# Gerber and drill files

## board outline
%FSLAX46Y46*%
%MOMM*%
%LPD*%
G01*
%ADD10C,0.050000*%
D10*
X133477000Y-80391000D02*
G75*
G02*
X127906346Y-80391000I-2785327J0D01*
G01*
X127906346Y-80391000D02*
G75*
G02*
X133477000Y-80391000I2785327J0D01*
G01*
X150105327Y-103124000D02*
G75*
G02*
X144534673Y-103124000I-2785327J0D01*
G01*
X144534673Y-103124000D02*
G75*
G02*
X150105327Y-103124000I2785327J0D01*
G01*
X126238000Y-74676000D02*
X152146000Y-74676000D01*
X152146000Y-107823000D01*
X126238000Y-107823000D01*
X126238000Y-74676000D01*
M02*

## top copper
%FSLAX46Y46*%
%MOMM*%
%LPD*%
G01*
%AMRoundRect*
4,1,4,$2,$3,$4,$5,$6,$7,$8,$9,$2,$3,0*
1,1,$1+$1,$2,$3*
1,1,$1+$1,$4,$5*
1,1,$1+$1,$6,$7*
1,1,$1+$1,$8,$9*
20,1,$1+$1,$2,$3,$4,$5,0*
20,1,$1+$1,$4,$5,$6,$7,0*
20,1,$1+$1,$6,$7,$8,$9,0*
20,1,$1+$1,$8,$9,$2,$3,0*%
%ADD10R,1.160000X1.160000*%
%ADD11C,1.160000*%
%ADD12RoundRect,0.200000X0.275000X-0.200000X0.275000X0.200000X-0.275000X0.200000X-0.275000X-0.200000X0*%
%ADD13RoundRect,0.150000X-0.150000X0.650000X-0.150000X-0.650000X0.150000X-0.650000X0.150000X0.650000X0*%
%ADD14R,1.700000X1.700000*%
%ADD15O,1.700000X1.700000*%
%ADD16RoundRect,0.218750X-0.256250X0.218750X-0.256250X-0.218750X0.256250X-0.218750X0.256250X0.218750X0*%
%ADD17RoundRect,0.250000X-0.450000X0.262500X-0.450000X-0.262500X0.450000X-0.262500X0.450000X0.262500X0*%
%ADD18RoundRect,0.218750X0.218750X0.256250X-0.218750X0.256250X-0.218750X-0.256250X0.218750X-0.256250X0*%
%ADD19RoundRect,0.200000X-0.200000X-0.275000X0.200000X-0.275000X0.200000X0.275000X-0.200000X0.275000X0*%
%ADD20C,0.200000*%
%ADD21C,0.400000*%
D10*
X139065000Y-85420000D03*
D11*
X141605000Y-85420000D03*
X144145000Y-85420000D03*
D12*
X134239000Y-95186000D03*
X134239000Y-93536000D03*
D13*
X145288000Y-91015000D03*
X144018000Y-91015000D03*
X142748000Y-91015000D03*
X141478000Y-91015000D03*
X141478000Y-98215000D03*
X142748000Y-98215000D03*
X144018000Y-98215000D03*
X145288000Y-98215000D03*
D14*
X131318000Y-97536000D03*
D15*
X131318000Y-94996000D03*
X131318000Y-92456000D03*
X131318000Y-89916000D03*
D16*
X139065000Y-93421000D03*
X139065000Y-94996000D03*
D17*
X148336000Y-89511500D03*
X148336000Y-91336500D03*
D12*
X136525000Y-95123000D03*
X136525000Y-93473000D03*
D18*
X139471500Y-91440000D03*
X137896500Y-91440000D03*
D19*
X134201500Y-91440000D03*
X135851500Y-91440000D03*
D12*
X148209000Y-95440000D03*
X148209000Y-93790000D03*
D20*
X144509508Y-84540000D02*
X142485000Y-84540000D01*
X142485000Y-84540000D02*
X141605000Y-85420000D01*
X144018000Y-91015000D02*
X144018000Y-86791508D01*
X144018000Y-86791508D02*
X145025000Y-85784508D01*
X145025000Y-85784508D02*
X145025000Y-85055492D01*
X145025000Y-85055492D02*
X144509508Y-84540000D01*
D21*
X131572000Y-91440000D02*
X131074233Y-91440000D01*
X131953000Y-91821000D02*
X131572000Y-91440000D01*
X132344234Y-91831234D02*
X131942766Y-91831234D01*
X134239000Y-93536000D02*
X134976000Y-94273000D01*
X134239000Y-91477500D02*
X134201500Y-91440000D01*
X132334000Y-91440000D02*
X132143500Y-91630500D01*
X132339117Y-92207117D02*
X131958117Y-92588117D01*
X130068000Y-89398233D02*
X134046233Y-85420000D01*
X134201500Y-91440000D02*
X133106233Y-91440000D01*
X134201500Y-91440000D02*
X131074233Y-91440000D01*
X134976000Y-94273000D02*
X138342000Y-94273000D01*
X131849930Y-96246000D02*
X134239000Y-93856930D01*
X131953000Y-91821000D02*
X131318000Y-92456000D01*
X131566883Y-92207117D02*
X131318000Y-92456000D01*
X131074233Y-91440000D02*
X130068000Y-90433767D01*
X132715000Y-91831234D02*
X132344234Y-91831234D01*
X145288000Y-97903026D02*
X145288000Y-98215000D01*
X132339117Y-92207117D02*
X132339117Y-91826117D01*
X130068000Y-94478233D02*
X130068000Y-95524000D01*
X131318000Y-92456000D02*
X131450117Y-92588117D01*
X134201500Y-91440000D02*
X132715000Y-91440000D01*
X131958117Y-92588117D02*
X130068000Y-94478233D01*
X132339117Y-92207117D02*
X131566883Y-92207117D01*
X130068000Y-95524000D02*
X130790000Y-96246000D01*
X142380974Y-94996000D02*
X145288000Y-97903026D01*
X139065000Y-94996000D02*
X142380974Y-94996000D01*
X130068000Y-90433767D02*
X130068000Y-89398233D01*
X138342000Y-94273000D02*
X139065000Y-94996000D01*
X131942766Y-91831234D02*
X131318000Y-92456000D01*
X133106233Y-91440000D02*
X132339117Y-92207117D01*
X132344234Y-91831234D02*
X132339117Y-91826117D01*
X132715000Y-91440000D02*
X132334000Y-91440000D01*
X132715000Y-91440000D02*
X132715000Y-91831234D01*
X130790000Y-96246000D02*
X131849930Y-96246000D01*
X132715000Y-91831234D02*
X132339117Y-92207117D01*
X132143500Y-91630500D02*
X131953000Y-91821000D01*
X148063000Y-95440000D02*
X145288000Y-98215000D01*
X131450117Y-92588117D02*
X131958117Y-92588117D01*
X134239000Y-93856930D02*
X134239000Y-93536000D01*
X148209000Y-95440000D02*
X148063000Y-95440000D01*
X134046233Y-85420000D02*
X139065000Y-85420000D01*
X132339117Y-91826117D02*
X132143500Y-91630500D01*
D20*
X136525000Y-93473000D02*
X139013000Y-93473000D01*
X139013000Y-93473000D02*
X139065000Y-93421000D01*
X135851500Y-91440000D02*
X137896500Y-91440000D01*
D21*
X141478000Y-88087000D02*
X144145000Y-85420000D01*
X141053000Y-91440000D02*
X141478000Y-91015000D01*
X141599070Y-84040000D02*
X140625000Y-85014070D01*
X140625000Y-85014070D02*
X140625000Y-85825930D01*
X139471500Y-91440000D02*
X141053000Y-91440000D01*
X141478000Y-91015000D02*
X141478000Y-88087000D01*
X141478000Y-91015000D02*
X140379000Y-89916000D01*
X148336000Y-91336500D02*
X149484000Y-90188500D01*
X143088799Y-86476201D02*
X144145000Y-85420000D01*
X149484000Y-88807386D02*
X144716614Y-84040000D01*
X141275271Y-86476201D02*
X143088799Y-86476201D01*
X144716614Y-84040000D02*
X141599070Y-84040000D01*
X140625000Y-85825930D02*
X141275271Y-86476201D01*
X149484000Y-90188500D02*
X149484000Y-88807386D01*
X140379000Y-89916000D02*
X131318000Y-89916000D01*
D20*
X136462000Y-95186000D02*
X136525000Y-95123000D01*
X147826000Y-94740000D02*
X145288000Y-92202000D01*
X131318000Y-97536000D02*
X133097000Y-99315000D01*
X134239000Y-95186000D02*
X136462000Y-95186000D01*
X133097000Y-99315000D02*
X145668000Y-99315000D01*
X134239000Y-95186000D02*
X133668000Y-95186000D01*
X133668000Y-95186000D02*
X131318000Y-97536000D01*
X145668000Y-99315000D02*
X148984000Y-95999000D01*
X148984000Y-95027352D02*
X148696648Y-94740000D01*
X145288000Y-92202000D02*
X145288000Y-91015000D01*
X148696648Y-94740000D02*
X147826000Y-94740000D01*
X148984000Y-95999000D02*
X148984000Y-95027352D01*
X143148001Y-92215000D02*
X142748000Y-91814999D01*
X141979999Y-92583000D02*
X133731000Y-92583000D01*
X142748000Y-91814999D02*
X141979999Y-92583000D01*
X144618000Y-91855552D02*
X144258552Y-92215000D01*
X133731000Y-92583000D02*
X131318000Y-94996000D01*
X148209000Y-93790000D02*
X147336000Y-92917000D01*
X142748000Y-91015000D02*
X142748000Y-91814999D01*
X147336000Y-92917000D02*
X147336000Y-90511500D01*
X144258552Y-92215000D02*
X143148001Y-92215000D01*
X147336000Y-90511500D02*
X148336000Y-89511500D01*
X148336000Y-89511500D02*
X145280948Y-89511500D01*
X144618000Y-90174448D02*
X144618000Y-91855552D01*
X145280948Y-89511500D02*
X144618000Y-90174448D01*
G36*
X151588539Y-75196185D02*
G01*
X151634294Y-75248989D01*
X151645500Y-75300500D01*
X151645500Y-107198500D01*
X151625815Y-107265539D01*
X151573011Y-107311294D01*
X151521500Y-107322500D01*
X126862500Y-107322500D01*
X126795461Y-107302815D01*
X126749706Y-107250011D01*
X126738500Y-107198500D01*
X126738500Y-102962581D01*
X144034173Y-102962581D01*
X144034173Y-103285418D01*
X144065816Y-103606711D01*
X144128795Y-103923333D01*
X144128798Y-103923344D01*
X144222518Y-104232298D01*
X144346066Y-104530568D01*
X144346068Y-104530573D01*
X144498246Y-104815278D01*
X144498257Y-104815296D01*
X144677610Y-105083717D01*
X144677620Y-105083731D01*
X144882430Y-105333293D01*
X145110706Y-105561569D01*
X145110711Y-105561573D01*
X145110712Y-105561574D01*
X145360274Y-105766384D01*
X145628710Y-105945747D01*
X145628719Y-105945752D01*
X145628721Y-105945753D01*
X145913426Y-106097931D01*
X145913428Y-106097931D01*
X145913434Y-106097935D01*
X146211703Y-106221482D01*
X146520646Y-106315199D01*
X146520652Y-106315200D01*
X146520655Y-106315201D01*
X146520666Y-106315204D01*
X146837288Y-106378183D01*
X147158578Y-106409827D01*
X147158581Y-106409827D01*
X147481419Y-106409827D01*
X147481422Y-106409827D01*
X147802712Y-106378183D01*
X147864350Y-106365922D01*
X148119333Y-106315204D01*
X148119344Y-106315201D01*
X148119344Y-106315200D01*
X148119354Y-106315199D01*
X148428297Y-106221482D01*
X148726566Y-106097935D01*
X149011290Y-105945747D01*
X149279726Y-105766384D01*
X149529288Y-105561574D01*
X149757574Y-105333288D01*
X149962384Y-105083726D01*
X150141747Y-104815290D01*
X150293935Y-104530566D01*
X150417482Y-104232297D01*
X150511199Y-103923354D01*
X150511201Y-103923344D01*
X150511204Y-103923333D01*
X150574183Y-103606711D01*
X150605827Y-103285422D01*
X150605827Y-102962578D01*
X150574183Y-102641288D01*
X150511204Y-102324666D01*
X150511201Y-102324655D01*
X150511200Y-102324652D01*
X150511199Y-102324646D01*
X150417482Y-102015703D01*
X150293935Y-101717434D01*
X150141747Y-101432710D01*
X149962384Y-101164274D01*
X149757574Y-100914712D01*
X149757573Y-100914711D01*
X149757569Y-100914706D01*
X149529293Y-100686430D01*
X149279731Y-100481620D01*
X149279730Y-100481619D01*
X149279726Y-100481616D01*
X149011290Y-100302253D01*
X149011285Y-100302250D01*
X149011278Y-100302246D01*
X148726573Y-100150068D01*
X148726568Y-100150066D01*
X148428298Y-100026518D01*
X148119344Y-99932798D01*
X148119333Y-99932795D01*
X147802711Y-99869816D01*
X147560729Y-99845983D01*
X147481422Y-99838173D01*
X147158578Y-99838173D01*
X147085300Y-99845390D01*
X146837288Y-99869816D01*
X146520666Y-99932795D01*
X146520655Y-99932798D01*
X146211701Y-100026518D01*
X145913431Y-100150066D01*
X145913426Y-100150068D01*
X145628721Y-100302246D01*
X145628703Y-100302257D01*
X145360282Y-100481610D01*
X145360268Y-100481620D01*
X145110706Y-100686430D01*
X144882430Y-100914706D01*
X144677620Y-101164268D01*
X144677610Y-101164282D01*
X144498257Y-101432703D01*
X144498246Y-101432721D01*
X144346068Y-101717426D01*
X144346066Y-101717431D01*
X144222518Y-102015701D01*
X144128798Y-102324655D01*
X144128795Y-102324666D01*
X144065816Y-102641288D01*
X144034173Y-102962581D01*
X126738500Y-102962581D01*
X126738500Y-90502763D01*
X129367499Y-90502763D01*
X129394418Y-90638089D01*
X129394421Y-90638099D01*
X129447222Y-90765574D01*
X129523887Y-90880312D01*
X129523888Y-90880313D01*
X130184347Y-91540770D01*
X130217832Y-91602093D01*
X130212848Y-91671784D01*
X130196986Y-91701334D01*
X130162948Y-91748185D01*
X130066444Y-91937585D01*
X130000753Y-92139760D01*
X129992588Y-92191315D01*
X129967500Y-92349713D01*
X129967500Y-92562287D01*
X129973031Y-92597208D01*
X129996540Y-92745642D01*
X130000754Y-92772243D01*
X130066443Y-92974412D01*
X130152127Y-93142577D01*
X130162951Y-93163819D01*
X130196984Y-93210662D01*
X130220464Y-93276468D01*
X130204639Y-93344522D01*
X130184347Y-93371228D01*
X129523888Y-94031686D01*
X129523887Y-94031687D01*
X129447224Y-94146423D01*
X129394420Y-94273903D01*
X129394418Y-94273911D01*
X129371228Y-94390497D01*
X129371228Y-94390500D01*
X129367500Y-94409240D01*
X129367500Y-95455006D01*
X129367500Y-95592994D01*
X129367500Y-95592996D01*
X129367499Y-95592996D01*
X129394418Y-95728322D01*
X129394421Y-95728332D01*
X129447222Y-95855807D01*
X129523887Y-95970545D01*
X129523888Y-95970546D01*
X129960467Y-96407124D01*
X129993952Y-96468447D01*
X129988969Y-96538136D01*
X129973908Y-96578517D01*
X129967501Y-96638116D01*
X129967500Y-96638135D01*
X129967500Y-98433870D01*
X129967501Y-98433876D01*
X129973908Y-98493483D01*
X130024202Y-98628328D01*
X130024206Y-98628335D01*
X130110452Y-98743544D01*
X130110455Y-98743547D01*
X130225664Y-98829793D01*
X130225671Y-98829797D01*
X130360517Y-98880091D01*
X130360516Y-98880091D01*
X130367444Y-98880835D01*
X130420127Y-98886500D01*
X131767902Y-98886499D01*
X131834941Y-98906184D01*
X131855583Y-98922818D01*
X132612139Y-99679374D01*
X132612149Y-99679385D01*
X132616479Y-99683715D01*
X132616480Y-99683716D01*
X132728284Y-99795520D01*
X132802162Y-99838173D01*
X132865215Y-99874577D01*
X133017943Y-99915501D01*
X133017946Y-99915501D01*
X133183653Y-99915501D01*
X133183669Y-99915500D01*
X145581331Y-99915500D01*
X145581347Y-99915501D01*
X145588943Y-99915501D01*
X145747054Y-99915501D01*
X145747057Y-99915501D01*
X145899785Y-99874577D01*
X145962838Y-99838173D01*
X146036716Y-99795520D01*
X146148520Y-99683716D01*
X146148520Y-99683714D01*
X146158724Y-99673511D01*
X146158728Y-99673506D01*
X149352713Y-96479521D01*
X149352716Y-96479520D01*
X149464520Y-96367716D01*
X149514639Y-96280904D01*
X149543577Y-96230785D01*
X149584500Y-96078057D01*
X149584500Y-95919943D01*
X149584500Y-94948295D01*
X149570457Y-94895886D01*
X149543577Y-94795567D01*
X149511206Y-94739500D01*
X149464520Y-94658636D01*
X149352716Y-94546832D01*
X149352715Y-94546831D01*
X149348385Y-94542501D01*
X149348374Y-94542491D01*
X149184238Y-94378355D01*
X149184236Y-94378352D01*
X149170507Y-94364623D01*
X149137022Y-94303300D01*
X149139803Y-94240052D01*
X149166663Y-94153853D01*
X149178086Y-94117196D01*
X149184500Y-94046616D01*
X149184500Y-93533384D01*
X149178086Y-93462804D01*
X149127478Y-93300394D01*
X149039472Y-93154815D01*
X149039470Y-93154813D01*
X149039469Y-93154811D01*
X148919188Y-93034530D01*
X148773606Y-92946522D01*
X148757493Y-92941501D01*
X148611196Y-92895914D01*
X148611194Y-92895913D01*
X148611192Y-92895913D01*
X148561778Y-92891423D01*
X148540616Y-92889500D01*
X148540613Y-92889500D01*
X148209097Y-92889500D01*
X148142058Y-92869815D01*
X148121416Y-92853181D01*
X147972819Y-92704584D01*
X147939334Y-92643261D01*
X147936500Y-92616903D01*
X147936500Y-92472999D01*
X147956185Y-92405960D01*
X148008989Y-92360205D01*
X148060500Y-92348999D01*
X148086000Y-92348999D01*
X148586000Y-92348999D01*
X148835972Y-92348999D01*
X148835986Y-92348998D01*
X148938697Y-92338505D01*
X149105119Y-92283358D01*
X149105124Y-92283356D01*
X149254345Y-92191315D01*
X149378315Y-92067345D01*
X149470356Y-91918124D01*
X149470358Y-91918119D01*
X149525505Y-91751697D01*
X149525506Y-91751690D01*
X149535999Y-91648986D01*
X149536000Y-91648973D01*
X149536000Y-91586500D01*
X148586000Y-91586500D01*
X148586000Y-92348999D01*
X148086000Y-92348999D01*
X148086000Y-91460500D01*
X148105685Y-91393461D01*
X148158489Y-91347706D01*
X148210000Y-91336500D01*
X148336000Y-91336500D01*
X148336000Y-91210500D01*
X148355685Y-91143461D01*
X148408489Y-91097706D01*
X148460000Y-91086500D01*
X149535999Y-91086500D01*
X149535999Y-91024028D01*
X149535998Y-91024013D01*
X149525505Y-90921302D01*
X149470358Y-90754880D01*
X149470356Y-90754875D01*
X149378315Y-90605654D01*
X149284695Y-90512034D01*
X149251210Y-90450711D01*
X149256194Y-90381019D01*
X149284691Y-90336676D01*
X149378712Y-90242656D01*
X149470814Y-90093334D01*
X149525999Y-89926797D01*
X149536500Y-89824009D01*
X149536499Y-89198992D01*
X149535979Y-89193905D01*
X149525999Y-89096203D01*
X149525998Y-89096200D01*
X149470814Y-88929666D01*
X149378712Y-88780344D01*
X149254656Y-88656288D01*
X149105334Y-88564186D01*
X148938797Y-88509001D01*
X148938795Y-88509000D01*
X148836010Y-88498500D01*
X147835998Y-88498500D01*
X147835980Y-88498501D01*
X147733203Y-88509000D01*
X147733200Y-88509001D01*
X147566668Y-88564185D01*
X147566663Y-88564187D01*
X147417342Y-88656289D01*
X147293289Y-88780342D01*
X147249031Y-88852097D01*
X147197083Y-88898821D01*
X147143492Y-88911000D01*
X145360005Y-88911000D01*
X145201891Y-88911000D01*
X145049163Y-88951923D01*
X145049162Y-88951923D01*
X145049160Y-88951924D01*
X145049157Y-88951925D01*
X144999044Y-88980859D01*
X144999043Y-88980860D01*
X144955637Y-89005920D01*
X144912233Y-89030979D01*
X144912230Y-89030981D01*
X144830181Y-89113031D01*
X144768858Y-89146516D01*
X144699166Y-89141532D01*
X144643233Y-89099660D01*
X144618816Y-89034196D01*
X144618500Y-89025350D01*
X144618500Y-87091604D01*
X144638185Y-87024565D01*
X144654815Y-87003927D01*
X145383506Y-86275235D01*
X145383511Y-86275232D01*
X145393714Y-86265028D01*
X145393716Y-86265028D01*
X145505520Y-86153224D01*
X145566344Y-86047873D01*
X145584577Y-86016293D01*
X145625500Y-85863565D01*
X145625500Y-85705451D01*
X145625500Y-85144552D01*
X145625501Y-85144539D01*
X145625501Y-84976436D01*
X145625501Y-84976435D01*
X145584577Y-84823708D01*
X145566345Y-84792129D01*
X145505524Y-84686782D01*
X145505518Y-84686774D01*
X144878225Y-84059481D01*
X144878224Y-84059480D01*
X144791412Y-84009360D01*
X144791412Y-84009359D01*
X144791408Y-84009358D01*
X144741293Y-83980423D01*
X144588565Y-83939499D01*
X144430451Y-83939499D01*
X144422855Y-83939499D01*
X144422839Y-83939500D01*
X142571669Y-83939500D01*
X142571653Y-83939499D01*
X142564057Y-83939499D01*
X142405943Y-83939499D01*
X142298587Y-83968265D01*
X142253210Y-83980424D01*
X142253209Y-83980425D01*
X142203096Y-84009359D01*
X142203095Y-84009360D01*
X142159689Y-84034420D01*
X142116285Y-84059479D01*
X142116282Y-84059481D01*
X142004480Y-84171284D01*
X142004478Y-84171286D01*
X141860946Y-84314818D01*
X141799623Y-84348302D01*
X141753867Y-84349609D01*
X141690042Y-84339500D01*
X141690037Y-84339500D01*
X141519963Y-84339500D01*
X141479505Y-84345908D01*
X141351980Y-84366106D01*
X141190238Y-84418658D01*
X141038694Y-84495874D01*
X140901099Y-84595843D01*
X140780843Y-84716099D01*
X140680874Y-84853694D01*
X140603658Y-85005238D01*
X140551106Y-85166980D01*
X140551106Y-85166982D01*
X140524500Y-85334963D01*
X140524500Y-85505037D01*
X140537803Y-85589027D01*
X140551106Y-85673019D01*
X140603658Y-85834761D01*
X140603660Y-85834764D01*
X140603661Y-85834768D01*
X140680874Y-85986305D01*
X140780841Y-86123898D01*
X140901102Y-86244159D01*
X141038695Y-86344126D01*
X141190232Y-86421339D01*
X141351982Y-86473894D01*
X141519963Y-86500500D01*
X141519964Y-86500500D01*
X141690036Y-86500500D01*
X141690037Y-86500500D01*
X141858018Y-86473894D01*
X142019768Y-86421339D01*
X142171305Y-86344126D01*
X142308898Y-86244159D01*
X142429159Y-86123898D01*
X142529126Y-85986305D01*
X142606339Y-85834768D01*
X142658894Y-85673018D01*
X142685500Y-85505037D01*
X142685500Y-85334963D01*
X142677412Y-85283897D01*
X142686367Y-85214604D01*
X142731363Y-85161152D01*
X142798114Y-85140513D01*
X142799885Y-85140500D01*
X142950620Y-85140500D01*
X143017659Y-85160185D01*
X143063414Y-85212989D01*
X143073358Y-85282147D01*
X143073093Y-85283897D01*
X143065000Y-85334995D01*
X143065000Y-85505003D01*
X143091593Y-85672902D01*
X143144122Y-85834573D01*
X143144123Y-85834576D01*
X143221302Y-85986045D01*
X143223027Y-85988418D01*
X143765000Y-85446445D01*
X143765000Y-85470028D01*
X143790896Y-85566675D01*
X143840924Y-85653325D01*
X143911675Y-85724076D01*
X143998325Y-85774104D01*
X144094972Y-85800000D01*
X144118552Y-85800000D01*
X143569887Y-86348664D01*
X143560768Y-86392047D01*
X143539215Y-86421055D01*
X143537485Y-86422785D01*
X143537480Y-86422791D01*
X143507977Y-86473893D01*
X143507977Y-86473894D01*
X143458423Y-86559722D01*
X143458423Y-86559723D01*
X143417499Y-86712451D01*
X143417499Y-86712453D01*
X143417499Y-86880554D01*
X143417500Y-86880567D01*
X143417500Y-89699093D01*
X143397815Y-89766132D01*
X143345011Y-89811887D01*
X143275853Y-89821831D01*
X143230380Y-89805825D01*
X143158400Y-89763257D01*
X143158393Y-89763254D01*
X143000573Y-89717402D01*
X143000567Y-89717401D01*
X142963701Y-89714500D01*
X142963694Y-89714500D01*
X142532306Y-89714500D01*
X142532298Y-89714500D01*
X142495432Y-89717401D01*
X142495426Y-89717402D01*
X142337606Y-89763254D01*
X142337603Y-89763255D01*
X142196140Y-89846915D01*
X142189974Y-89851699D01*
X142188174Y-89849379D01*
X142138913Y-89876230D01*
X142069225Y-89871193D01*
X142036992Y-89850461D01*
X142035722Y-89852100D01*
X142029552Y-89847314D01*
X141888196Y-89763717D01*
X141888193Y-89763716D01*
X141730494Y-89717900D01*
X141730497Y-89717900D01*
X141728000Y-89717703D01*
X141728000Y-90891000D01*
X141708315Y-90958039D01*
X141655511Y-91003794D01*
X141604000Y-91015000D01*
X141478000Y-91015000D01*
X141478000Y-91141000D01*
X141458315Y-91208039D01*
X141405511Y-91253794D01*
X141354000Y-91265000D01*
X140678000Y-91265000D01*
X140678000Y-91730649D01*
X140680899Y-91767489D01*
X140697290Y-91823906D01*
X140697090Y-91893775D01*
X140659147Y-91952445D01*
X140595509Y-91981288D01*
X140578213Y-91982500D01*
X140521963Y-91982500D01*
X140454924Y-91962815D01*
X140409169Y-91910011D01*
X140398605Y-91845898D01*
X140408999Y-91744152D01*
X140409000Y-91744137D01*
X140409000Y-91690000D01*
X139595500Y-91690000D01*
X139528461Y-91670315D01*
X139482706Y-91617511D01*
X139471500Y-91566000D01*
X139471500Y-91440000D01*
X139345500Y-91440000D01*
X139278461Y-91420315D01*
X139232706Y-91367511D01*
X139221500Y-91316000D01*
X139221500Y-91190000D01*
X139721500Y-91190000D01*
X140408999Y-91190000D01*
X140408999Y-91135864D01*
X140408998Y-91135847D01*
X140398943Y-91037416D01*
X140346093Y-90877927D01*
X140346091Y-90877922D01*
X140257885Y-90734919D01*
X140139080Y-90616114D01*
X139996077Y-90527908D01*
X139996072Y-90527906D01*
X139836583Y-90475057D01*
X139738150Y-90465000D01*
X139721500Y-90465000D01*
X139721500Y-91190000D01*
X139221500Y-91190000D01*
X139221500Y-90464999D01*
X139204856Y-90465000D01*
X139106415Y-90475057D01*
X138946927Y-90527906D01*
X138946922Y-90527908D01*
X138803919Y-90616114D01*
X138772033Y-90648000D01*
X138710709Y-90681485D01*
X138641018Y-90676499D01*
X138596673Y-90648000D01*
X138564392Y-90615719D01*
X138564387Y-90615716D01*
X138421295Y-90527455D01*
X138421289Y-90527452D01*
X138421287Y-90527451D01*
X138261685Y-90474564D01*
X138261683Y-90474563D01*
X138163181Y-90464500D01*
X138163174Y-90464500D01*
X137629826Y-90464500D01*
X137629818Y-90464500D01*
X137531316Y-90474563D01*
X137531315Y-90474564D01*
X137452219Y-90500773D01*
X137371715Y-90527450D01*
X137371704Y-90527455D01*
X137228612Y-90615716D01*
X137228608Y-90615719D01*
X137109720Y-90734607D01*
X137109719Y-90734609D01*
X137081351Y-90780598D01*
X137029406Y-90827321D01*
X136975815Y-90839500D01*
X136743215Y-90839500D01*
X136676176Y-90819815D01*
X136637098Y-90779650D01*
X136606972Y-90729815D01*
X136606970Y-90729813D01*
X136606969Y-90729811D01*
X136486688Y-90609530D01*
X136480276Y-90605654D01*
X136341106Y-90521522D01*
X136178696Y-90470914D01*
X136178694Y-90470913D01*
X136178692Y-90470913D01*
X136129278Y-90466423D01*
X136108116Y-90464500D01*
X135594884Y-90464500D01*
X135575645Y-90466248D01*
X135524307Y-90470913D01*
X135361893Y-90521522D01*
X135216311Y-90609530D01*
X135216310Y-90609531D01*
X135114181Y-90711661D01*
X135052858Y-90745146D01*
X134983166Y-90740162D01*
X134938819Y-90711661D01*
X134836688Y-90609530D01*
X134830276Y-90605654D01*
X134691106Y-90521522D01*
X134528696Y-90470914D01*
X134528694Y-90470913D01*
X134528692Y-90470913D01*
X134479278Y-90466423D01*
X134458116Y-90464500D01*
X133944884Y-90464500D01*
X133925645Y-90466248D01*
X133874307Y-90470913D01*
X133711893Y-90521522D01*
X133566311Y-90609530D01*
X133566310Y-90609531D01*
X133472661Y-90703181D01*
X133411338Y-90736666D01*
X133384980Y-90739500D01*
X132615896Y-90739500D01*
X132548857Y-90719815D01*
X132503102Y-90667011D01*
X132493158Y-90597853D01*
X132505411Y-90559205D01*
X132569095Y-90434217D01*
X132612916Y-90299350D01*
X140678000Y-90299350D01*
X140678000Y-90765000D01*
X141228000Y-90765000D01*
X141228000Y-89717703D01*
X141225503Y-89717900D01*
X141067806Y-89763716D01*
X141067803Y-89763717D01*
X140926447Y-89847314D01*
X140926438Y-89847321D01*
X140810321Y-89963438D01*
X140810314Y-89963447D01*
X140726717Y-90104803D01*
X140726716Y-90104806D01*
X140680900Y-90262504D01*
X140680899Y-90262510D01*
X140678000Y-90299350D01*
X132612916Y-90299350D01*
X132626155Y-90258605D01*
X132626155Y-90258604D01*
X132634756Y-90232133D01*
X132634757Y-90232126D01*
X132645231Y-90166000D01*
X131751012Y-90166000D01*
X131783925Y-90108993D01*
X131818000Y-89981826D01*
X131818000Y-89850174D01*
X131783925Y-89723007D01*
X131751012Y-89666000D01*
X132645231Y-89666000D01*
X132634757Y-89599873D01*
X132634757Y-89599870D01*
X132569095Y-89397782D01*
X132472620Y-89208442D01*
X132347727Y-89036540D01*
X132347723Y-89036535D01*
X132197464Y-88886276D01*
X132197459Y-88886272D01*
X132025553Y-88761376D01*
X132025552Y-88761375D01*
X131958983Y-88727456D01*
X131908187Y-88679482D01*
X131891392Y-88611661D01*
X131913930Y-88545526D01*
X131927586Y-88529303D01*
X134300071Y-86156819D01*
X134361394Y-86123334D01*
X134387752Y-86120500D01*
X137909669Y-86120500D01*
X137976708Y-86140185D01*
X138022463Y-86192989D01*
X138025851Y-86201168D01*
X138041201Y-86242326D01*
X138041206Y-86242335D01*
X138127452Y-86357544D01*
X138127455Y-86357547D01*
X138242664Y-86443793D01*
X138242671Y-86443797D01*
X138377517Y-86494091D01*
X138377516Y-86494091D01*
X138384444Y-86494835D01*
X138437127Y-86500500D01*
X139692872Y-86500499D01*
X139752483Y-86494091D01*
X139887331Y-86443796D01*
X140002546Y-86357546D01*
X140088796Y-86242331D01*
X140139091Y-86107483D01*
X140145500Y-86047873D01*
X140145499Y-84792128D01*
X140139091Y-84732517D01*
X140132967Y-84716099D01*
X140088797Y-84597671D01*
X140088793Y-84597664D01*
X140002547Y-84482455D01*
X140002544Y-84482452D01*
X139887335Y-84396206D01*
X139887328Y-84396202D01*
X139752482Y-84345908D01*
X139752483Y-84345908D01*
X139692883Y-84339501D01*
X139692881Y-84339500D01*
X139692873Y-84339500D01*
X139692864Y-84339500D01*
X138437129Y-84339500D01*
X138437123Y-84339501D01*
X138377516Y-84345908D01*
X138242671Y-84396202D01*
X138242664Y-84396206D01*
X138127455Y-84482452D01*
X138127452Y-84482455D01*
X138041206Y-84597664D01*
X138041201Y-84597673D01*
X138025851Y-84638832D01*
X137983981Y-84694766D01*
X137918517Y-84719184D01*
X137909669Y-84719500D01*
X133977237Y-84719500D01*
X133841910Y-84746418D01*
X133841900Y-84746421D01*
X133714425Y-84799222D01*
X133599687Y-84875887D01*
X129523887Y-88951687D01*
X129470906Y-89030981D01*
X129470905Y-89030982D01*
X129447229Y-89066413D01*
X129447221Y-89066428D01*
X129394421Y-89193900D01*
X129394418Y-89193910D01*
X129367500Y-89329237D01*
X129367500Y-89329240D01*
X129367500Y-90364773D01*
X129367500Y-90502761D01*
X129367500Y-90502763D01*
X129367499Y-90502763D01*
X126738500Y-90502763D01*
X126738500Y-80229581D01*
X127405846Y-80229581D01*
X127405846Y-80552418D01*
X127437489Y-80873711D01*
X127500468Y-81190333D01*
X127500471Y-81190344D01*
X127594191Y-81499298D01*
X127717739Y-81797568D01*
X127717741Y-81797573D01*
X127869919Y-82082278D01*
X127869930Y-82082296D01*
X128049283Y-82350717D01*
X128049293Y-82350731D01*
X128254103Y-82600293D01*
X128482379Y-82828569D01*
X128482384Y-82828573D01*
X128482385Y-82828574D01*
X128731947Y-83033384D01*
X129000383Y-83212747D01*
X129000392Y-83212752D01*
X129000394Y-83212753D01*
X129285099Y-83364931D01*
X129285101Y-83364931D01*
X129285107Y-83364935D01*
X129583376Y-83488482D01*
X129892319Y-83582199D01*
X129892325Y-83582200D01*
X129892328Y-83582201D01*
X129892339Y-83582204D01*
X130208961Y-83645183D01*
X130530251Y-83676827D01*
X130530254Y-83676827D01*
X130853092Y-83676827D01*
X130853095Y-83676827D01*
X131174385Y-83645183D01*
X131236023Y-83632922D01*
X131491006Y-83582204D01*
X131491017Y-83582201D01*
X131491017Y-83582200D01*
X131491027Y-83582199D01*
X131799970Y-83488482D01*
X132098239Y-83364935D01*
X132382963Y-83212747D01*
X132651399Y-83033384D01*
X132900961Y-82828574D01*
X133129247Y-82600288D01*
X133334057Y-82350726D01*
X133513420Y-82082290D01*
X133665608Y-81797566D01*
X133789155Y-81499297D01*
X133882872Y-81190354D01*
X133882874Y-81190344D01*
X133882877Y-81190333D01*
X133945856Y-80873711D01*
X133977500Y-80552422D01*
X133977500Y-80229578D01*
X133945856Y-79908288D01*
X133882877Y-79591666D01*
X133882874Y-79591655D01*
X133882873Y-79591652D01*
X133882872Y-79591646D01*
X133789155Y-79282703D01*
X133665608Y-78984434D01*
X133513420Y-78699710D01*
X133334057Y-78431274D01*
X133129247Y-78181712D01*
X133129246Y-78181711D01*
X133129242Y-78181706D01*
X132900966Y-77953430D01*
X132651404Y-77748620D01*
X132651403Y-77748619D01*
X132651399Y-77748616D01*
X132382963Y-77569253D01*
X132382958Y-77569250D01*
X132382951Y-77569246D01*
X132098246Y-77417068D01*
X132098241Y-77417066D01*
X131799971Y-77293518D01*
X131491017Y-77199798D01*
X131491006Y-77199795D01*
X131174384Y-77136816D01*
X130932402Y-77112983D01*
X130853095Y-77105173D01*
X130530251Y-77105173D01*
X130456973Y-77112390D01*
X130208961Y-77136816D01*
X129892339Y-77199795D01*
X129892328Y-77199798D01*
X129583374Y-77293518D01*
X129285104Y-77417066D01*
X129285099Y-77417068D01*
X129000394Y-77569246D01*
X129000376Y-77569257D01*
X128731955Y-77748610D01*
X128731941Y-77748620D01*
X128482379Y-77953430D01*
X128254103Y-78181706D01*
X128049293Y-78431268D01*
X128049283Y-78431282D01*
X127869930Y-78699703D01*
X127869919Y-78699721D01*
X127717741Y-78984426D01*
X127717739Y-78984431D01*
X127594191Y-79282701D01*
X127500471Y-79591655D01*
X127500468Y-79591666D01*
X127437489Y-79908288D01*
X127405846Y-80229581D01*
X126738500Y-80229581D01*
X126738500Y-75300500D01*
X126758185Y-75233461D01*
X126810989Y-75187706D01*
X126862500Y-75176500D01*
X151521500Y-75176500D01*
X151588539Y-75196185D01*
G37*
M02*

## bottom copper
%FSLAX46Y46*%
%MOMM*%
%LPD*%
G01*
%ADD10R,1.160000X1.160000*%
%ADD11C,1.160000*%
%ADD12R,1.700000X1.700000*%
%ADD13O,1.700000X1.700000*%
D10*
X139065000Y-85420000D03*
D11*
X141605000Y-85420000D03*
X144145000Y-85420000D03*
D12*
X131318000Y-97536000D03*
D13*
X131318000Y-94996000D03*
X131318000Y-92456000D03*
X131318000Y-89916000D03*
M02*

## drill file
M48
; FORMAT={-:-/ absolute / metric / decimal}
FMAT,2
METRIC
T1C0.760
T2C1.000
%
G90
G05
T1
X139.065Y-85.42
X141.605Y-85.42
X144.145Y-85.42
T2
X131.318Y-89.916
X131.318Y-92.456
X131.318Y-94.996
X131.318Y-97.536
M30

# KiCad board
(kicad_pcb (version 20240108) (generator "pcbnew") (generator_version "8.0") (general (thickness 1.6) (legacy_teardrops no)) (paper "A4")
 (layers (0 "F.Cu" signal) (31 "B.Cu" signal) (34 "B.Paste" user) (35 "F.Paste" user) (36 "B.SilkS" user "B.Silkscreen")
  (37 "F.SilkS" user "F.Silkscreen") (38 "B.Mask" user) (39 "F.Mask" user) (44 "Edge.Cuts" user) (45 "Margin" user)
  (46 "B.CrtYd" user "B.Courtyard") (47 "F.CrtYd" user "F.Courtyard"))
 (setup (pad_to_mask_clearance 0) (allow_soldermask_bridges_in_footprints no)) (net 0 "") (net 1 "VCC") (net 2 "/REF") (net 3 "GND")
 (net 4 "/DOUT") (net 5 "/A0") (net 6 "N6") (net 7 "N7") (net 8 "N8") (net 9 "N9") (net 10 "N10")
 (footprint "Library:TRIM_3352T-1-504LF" (layer "F.Cu") (at 141.605 82.55)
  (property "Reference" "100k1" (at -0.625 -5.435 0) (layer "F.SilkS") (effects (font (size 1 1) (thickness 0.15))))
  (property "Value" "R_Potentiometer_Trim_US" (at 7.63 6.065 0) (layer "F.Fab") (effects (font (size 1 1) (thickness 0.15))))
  (pad "1" thru_hole rect (at -2.54 2.87) (size 1.16 1.16) (drill 0.76) (layers "*.Cu" "*.Mask") (remove_unused_layers no) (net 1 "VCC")
   (solder_mask_margin 0.102))
  (pad "2" thru_hole circle (at 0 2.87) (size 1.16 1.16) (drill 0.76) (layers "*.Cu" "*.Mask") (remove_unused_layers no) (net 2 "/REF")
   (solder_mask_margin 0.102))
  (pad "3" thru_hole circle (at 2.54 2.87) (size 1.16 1.16) (drill 0.76) (layers "*.Cu" "*.Mask") (remove_unused_layers no) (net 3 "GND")
   (solder_mask_margin 0.102)))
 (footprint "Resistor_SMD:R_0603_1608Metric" (layer "F.Cu") (at 134.239 94.361 90)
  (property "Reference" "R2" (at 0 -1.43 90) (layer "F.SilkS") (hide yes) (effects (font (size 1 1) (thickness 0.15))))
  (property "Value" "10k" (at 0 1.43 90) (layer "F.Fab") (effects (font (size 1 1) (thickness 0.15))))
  (pad "1" smd roundrect (at -0.825 0 90) (size 0.8 0.95) (layers "F.Cu" "F.Paste" "F.Mask") (roundrect_rratio 0.25) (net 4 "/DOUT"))
  (pad "2" smd roundrect (at 0.825 0 90) (size 0.8 0.95) (layers "F.Cu" "F.Paste" "F.Mask") (roundrect_rratio 0.25) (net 1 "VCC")))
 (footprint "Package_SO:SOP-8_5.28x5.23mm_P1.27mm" (layer "F.Cu") (at 143.383 94.615 -90)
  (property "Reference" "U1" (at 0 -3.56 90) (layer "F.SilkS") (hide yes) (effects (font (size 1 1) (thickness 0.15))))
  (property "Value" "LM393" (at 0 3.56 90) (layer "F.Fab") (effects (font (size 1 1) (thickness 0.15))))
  (pad "1" smd roundrect (at -3.6 -1.905 270) (size 1.6 0.6) (layers "F.Cu" "F.Paste" "F.Mask") (roundrect_rratio 0.25) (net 4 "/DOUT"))
  (pad "2" smd roundrect (at -3.6 -0.635 270) (size 1.6 0.6) (layers "F.Cu" "F.Paste" "F.Mask") (roundrect_rratio 0.25) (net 2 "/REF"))
  (pad "3" smd roundrect (at -3.6 0.635 270) (size 1.6 0.6) (layers "F.Cu" "F.Paste" "F.Mask") (roundrect_rratio 0.25) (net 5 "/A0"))
  (pad "4" smd roundrect (at -3.6 1.905 270) (size 1.6 0.6) (layers "F.Cu" "F.Paste" "F.Mask") (roundrect_rratio 0.25) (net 3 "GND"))
  (pad "5" smd roundrect (at 3.6 1.905 270) (size 1.6 0.6) (layers "F.Cu" "F.Paste" "F.Mask") (roundrect_rratio 0.25) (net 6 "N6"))
  (pad "6" smd roundrect (at 3.6 0.635 270) (size 1.6 0.6) (layers "F.Cu" "F.Paste" "F.Mask") (roundrect_rratio 0.25) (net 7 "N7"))
  (pad "7" smd roundrect (at 3.6 -0.635 270) (size 1.6 0.6) (layers "F.Cu" "F.Paste" "F.Mask") (roundrect_rratio 0.25) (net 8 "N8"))
  (pad "8" smd roundrect (at 3.6 -1.905 270) (size 1.6 0.6) (layers "F.Cu" "F.Paste" "F.Mask") (roundrect_rratio 0.25) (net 1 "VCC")))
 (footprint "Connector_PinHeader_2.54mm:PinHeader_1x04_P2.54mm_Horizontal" (layer "F.Cu") (at 131.318 97.536 180)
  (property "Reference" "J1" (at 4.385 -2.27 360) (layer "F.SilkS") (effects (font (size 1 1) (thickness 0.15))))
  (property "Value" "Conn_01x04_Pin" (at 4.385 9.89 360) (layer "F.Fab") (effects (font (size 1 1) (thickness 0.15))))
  (pad "1" thru_hole rect (at 0 0 180) (size 1.7 1.7) (drill 1) (layers "*.Cu" "*.Mask") (remove_unused_layers no) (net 4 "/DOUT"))
  (pad "2" thru_hole oval (at 0 2.54 180) (size 1.7 1.7) (drill 1) (layers "*.Cu" "*.Mask") (remove_unused_layers no) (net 5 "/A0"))
  (pad "3" thru_hole oval (at 0 5.08 180) (size 1.7 1.7) (drill 1) (layers "*.Cu" "*.Mask") (remove_unused_layers no) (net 1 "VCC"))
  (pad "4" thru_hole oval (at 0 7.62 180) (size 1.7 1.7) (drill 1) (layers "*.Cu" "*.Mask") (remove_unused_layers no) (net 3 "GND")))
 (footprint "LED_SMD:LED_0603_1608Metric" (layer "F.Cu") (at 139.065 94.2085 -90)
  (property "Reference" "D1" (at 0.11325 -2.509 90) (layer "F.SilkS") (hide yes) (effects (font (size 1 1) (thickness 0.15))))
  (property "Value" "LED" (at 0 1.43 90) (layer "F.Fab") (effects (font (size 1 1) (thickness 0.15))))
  (pad "1" smd roundrect (at -0.7875 0 270) (size 0.875 0.95) (layers "F.Cu" "F.Paste" "F.Mask") (roundrect_rratio 0.25) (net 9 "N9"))
  (pad "2" smd roundrect (at 0.7875 0 270) (size 0.875 0.95) (layers "F.Cu" "F.Paste" "F.Mask") (roundrect_rratio 0.25) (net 1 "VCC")))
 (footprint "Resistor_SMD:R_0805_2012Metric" (layer "F.Cu") (at 148.336 90.424 -90)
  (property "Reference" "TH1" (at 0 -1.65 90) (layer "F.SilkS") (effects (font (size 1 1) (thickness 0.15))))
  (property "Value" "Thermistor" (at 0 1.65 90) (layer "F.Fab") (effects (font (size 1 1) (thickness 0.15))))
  (pad "1" smd roundrect (at -0.9125 0 270) (size 1.025 1.4) (layers "F.Cu" "F.Paste" "F.Mask") (roundrect_rratio 0.243902) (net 5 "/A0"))
  (pad "2" smd roundrect (at 0.9125 0 270) (size 1.025 1.4) (layers "F.Cu" "F.Paste" "F.Mask") (roundrect_rratio 0.243902) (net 3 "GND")))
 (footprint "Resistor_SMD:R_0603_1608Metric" (layer "F.Cu") (at 136.525 94.298 90)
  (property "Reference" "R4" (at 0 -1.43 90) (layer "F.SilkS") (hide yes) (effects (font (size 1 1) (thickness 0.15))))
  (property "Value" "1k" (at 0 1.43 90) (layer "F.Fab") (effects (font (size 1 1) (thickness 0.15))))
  (pad "1" smd roundrect (at -0.825 0 90) (size 0.8 0.95) (layers "F.Cu" "F.Paste" "F.Mask") (roundrect_rratio 0.25) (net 4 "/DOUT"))
  (pad "2" smd roundrect (at 0.825 0 90) (size 0.8 0.95) (layers "F.Cu" "F.Paste" "F.Mask") (roundrect_rratio 0.25) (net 9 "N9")))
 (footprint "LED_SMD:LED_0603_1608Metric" (layer "F.Cu") (at 138.684 91.44 180)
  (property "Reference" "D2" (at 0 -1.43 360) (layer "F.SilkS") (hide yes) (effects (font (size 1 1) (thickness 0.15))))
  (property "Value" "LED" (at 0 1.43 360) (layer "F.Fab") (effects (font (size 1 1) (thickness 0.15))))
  (pad "1" smd roundrect (at -0.7875 0 180) (size 0.875 0.95) (layers "F.Cu" "F.Paste" "F.Mask") (roundrect_rratio 0.25) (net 3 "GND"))
  (pad "2" smd roundrect (at 0.7875 0 180) (size 0.875 0.95) (layers "F.Cu" "F.Paste" "F.Mask") (roundrect_rratio 0.25) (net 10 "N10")))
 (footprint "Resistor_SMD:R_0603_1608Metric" (layer "F.Cu") (at 135.0265 91.44)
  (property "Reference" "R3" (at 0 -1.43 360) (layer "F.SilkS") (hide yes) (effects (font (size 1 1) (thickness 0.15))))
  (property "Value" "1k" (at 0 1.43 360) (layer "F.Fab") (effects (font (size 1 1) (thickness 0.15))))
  (pad "1" smd roundrect (at -0.825 0) (size 0.8 0.95) (layers "F.Cu" "F.Paste" "F.Mask") (roundrect_rratio 0.25) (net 1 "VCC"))
  (pad "2" smd roundrect (at 0.825 0) (size 0.8 0.95) (layers "F.Cu" "F.Paste" "F.Mask") (roundrect_rratio 0.25) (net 10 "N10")))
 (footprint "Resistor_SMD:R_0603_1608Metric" (layer "F.Cu") (at 148.209 94.615 90)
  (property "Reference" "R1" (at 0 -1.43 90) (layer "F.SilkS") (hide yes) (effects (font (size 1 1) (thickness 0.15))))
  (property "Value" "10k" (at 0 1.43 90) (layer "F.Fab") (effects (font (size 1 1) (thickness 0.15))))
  (pad "1" smd roundrect (at -0.825 0 90) (size 0.8 0.95) (layers "F.Cu" "F.Paste" "F.Mask") (roundrect_rratio 0.25) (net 1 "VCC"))
  (pad "2" smd roundrect (at 0.825 0 90) (size 0.8 0.95) (layers "F.Cu" "F.Paste" "F.Mask") (roundrect_rratio 0.25) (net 5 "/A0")))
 (gr_circle (center 130.691673 80.391) (end 131.834673 77.851) (stroke (width 0.05) (type default)) (fill none) (layer "Edge.Cuts"))
 (gr_circle (center 147.32 103.124) (end 148.463 100.584) (stroke (width 0.05) (type default)) (fill none) (layer "Edge.Cuts"))
 (gr_rect (start 126.238 74.676) (end 152.146 107.823) (stroke (width 0.05) (type default)) (fill none) (layer "Edge.Cuts"))
 (segment (start 144.509508 84.54) (end 142.485 84.54) (width 0.2) (layer "F.Cu") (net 2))
 (segment (start 142.485 84.54) (end 141.605 85.42) (width 0.2) (layer "F.Cu") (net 2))
 (segment (start 144.018 91.015) (end 144.018 86.791508) (width 0.2) (layer "F.Cu") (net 2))
 (segment (start 144.018 86.791508) (end 145.025 85.784508) (width 0.2) (layer "F.Cu") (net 2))
 (segment (start 145.025 85.784508) (end 145.025 85.055492) (width 0.2) (layer "F.Cu") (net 2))
 (segment (start 145.025 85.055492) (end 144.509508 84.54) (width 0.2) (layer "F.Cu") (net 2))
 (segment (start 131.572 91.44) (end 131.074233 91.44) (width 0.4) (layer "F.Cu") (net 1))
 (segment (start 131.953 91.821) (end 131.572 91.44) (width 0.4) (layer "F.Cu") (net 1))
 (segment (start 132.344234 91.831234) (end 131.942766 91.831234) (width 0.4) (layer "F.Cu") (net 1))
 (segment (start 134.239 93.536) (end 134.976 94.273) (width 0.4) (layer "F.Cu") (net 1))
 (segment (start 134.239 91.4775) (end 134.2015 91.44) (width 0.4) (layer "F.Cu") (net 1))
 (segment (start 132.334 91.44) (end 132.1435 91.6305) (width 0.4) (layer "F.Cu") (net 1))
 (segment (start 132.339117 92.207117) (end 131.958117 92.588117) (width 0.4) (layer "F.Cu") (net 1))
 (segment (start 130.068 89.398233) (end 134.046233 85.42) (width 0.4) (layer "F.Cu") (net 1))
 (segment (start 134.2015 91.44) (end 133.106233 91.44) (width 0.4) (layer "F.Cu") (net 1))
 (segment (start 134.2015 91.44) (end 131.074233 91.44) (width 0.4) (layer "F.Cu") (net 1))
 (segment (start 134.976 94.273) (end 138.342 94.273) (width 0.4) (layer "F.Cu") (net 1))
 (segment (start 131.84993 96.246) (end 134.239 93.85693) (width 0.4) (layer "F.Cu") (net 1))
 (segment (start 131.953 91.821) (end 131.318 92.456) (width 0.4) (layer "F.Cu") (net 1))
 (segment (start 131.566883 92.207117) (end 131.318 92.456) (width 0.4) (layer "F.Cu") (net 1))
 (segment (start 131.074233 91.44) (end 130.068 90.433767) (width 0.4) (layer "F.Cu") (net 1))
 (segment (start 132.715 91.831234) (end 132.344234 91.831234) (width 0.4) (layer "F.Cu") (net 1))
 (segment (start 145.288 97.903026) (end 145.288 98.215) (width 0.4) (layer "F.Cu") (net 1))
 (segment (start 132.339117 92.207117) (end 132.339117 91.826117) (width 0.4) (layer "F.Cu") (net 1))
 (segment (start 130.068 94.478233) (end 130.068 95.524) (width 0.4) (layer "F.Cu") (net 1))
 (segment (start 131.318 92.456) (end 131.450117 92.588117) (width 0.4) (layer "F.Cu") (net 1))
 (segment (start 134.2015 91.44) (end 132.715 91.44) (width 0.4) (layer "F.Cu") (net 1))
 (segment (start 131.958117 92.588117) (end 130.068 94.478233) (width 0.4) (layer "F.Cu") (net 1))
 (segment (start 132.339117 92.207117) (end 131.566883 92.207117) (width 0.4) (layer "F.Cu") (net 1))
 (segment (start 130.068 95.524) (end 130.79 96.246) (width 0.4) (layer "F.Cu") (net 1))
 (segment (start 142.380974 94.996) (end 145.288 97.903026) (width 0.4) (layer "F.Cu") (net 1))
 (segment (start 139.065 94.996) (end 142.380974 94.996) (width 0.4) (layer "F.Cu") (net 1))
 (segment (start 130.068 90.433767) (end 130.068 89.398233) (width 0.4) (layer "F.Cu") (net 1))
 (segment (start 138.342 94.273) (end 139.065 94.996) (width 0.4) (layer "F.Cu") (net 1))
 (segment (start 131.942766 91.831234) (end 131.318 92.456) (width 0.4) (layer "F.Cu") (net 1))
 (segment (start 133.106233 91.44) (end 132.339117 92.207117) (width 0.4) (layer "F.Cu") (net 1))
 (segment (start 132.344234 91.831234) (end 132.339117 91.826117) (width 0.4) (layer "F.Cu") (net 1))
 (segment (start 132.715 91.44) (end 132.334 91.44) (width 0.4) (layer "F.Cu") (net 1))
 (segment (start 132.715 91.44) (end 132.715 91.831234) (width 0.4) (layer "F.Cu") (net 1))
 (segment (start 130.79 96.246) (end 131.84993 96.246) (width 0.4) (layer "F.Cu") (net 1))
 (segment (start 132.715 91.831234) (end 132.339117 92.207117) (width 0.4) (layer "F.Cu") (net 1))
 (segment (start 132.1435 91.6305) (end 131.953 91.821) (width 0.4) (layer "F.Cu") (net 1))
 (segment (start 148.063 95.44) (end 145.288 98.215) (width 0.4) (layer "F.Cu") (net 1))
 (segment (start 131.450117 92.588117) (end 131.958117 92.588117) (width 0.4) (layer "F.Cu") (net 1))
 (segment (start 134.239 93.85693) (end 134.239 93.536) (width 0.4) (layer "F.Cu") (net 1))
 (segment (start 148.209 95.44) (end 148.063 95.44) (width 0.4) (layer "F.Cu") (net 1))
 (segment (start 134.046233 85.42) (end 139.065 85.42) (width 0.4) (layer "F.Cu") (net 1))
 (segment (start 132.339117 91.826117) (end 132.1435 91.6305) (width 0.4) (layer "F.Cu") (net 1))
 (segment (start 136.525 93.473) (end 139.013 93.473) (width 0.2) (layer "F.Cu") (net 9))
 (segment (start 139.013 93.473) (end 139.065 93.421) (width 0.2) (layer "F.Cu") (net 9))
 (segment (start 135.8515 91.44) (end 137.8965 91.44) (width 0.2) (layer "F.Cu") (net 10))
 (segment (start 141.478 88.087) (end 144.145 85.42) (width 0.4) (layer "F.Cu") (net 3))
 (segment (start 141.053 91.44) (end 141.478 91.015) (width 0.4) (layer "F.Cu") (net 3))
 (segment (start 141.59907 84.04) (end 140.625 85.01407) (width 0.4) (layer "F.Cu") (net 3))
 (segment (start 140.625 85.01407) (end 140.625 85.82593) (width 0.4) (layer "F.Cu") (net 3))
 (segment (start 139.4715 91.44) (end 141.053 91.44) (width 0.4) (layer "F.Cu") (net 3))
 (segment (start 141.478 91.015) (end 141.478 88.087) (width 0.4) (layer "F.Cu") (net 3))
 (segment (start 141.478 91.015) (end 140.379 89.916) (width 0.4) (layer "F.Cu") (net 3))
 (segment (start 148.336 91.3365) (end 149.484 90.1885) (width 0.4) (layer "F.Cu") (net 3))
 (segment (start 143.088799 86.476201) (end 144.145 85.42) (width 0.4) (layer "F.Cu") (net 3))
 (segment (start 149.484 88.807386) (end 144.716614 84.04) (width 0.4) (layer "F.Cu") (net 3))
 (segment (start 141.275271 86.476201) (end 143.088799 86.476201) (width 0.4) (layer "F.Cu") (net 3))
 (segment (start 144.716614 84.04) (end 141.59907 84.04) (width 0.4) (layer "F.Cu") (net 3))
 (segment (start 140.625 85.82593) (end 141.275271 86.476201) (width 0.4) (layer "F.Cu") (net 3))
 (segment (start 149.484 90.1885) (end 149.484 88.807386) (width 0.4) (layer "F.Cu") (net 3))
 (segment (start 140.379 89.916) (end 131.318 89.916) (width 0.4) (layer "F.Cu") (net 3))
 (segment (start 136.462 95.186) (end 136.525 95.123) (width 0.2) (layer "F.Cu") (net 4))
 (segment (start 147.826 94.74) (end 145.288 92.202) (width 0.2) (layer "F.Cu") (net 4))
 (segment (start 131.318 97.536) (end 133.097 99.315) (width 0.2) (layer "F.Cu") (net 4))
 (segment (start 134.239 95.186) (end 136.462 95.186) (width 0.2) (layer "F.Cu") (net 4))
 (segment (start 133.097 99.315) (end 145.668 99.315) (width 0.2) (layer "F.Cu") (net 4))
 (segment (start 134.239 95.186) (end 133.668 95.186) (width 0.2) (layer "F.Cu") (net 4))
 (segment (start 133.668 95.186) (end 131.318 97.536) (width 0.2) (layer "F.Cu") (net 4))
 (segment (start 145.668 99.315) (end 148.984 95.999) (width 0.2) (layer "F.Cu") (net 4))
 (segment (start 148.984 95.027352) (end 148.696648 94.74) (width 0.2) (layer "F.Cu") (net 4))
 (segment (start 145.288 92.202) (end 145.288 91.015) (width 0.2) (layer "F.Cu") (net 4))
 (segment (start 148.696648 94.74) (end 147.826 94.74) (width 0.2) (layer "F.Cu") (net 4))
 (segment (start 148.984 95.999) (end 148.984 95.027352) (width 0.2) (layer "F.Cu") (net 4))
 (segment (start 143.148001 92.215) (end 142.748 91.814999) (width 0.2) (layer "F.Cu") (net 5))
 (segment (start 141.979999 92.583) (end 133.731 92.583) (width 0.2) (layer "F.Cu") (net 5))
 (segment (start 142.748 91.814999) (end 141.979999 92.583) (width 0.2) (layer "F.Cu") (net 5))
 (segment (start 144.618 91.855552) (end 144.258552 92.215) (width 0.2) (layer "F.Cu") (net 5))
 (segment (start 133.731 92.583) (end 131.318 94.996) (width 0.2) (layer "F.Cu") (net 5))
 (segment (start 148.209 93.79) (end 147.336 92.917) (width 0.2) (layer "F.Cu") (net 5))
 (segment (start 142.748 91.015) (end 142.748 91.814999) (width 0.2) (layer "F.Cu") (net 5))
 (segment (start 147.336 92.917) (end 147.336 90.5115) (width 0.2) (layer "F.Cu") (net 5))
 (segment (start 144.258552 92.215) (end 143.148001 92.215) (width 0.2) (layer "F.Cu") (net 5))
 (segment (start 147.336 90.5115) (end 148.336 89.5115) (width 0.2) (layer "F.Cu") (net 5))
 (segment (start 148.336 89.5115) (end 145.280948 89.5115) (width 0.2) (layer "F.Cu") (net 5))
 (segment (start 144.618 90.174448) (end 144.618 91.855552) (width 0.2) (layer "F.Cu") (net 5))
 (segment (start 145.280948 89.5115) (end 144.618 90.174448) (width 0.2) (layer "F.Cu") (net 5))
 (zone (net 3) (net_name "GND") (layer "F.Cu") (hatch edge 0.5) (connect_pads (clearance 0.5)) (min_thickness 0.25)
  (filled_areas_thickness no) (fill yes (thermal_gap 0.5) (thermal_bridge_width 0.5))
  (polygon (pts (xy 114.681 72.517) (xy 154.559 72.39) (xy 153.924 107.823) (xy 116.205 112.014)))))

